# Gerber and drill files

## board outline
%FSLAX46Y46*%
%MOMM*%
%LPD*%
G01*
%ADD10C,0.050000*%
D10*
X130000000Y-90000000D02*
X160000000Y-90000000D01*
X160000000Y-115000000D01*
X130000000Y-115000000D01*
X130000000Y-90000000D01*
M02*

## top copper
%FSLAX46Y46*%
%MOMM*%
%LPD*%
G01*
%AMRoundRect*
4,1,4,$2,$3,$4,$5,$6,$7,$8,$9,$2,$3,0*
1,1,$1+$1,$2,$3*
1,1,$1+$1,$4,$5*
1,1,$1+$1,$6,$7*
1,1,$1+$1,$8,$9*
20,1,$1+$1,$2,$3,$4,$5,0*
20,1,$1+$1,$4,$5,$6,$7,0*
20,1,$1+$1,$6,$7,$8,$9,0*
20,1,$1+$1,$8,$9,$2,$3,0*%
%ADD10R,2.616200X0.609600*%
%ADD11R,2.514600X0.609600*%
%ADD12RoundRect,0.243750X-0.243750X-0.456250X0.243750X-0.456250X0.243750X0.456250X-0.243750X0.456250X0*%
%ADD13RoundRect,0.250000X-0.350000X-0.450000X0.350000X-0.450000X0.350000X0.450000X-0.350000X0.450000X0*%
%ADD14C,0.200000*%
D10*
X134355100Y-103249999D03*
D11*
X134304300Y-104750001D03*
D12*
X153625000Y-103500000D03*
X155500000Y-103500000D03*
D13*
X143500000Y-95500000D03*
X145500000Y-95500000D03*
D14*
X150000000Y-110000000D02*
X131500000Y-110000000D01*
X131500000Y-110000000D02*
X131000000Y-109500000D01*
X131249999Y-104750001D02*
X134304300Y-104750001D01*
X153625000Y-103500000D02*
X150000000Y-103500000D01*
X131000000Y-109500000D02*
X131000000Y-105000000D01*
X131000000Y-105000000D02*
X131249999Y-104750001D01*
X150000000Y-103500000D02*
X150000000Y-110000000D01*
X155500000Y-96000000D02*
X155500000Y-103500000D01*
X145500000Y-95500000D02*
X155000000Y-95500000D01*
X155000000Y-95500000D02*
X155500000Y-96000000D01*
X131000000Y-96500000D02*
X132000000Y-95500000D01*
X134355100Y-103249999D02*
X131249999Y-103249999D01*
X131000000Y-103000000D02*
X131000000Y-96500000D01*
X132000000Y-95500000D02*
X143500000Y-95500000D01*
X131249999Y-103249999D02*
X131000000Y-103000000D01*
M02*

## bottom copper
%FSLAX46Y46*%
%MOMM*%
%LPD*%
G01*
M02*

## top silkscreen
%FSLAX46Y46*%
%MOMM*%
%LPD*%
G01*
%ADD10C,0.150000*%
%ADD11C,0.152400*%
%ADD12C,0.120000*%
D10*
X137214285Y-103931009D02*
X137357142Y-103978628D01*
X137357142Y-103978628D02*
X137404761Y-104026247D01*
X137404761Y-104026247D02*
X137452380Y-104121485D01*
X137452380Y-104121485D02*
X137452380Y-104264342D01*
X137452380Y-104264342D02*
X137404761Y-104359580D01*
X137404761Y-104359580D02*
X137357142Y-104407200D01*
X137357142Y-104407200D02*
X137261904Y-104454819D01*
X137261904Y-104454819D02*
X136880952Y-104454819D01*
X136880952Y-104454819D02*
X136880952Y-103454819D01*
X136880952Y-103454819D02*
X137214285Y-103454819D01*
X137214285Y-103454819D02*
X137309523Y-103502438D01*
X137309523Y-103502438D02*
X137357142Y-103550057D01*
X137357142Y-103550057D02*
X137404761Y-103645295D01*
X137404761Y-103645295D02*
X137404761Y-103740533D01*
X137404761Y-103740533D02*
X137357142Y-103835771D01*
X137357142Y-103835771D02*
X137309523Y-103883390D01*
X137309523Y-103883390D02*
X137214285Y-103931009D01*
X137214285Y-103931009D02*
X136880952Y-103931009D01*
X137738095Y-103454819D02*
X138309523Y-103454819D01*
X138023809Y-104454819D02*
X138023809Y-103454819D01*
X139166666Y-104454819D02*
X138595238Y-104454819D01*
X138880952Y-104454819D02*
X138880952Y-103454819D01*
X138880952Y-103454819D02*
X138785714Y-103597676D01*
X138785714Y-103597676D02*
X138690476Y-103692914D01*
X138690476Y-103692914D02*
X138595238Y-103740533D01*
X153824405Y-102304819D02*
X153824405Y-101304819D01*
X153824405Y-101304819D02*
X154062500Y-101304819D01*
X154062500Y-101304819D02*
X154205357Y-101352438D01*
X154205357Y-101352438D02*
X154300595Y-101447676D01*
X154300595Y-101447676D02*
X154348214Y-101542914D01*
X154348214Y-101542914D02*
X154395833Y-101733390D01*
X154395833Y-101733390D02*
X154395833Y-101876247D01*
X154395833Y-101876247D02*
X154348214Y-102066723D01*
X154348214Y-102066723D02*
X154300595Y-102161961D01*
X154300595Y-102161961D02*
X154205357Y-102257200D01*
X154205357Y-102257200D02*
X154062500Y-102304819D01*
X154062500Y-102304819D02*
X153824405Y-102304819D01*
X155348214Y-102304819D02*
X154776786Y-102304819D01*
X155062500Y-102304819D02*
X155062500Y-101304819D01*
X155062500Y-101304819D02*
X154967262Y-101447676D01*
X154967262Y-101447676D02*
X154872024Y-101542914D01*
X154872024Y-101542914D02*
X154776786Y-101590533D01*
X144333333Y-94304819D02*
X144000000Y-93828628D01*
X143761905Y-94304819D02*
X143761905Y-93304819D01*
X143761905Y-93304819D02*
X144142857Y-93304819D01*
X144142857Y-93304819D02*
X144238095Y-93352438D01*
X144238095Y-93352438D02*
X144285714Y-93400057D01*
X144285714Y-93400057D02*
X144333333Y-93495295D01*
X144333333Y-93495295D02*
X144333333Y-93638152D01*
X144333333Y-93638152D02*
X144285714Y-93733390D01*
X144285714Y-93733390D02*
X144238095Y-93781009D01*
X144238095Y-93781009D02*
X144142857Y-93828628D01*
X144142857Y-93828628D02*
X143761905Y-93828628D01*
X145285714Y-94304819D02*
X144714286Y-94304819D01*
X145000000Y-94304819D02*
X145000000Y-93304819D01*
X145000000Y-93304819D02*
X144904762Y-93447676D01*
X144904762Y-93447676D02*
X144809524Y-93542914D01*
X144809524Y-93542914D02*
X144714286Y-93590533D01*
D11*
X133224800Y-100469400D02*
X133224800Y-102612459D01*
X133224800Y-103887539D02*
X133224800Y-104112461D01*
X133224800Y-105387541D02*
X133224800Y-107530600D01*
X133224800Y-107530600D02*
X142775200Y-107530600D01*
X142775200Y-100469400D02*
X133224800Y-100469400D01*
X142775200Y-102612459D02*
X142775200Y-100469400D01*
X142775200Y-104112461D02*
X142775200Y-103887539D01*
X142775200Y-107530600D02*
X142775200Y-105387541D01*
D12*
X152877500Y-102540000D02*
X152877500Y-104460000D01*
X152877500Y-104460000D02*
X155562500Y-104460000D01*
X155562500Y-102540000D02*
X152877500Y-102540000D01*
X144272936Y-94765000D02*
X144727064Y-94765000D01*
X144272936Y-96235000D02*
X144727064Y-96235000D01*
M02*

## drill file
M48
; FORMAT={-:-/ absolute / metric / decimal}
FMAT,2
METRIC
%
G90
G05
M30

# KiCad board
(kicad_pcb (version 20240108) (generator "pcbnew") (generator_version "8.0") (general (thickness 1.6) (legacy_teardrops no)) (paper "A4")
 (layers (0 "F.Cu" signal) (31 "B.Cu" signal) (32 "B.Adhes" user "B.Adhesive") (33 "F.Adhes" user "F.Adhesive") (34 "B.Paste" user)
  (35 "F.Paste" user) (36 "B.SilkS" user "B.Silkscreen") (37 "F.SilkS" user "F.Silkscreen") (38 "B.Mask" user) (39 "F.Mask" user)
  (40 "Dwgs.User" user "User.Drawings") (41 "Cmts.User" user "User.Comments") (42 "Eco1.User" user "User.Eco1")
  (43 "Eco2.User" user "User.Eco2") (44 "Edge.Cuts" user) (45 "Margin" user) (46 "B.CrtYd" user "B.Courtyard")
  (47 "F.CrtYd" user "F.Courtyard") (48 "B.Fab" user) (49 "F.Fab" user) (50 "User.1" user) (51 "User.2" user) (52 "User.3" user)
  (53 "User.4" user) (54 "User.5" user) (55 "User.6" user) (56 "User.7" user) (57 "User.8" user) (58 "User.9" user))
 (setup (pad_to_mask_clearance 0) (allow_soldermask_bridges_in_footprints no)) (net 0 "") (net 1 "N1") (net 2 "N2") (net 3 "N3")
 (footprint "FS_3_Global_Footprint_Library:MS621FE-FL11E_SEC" (layer "F.Cu") (at 138 104)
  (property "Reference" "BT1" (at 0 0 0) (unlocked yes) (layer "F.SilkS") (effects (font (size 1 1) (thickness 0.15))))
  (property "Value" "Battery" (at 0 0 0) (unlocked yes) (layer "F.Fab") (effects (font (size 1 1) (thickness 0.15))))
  (fp_line (start -4.7752 -3.5306) (end -4.7752 -1.387541) (stroke (width 0.1524) (type solid)) (layer "F.SilkS"))
  (fp_line (start -4.7752 -0.112461) (end -4.7752 0.112461) (stroke (width 0.1524) (type solid)) (layer "F.SilkS"))
  (fp_line (start -4.7752 1.387541) (end -4.7752 3.5306) (stroke (width 0.1524) (type solid)) (layer "F.SilkS"))
  (fp_line (start -4.7752 3.5306) (end 4.7752 3.5306) (stroke (width 0.1524) (type solid)) (layer "F.SilkS"))
  (fp_line (start 4.7752 -3.5306) (end -4.7752 -3.5306) (stroke (width 0.1524) (type solid)) (layer "F.SilkS"))
  (fp_line (start 4.7752 -1.387541) (end 4.7752 -3.5306) (stroke (width 0.1524) (type solid)) (layer "F.SilkS"))
  (fp_line (start 4.7752 0.112461) (end 4.7752 -0.112461) (stroke (width 0.1524) (type solid)) (layer "F.SilkS"))
  (fp_line (start 4.7752 3.5306) (end 4.7752 1.387541) (stroke (width 0.1524) (type solid)) (layer "F.SilkS"))
  (pad "1" smd rect (at -3.6449 -0.750001) (size 2.6162 0.6096) (layers "F.Cu" "F.Paste" "F.Mask") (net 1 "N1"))
  (pad "2" smd rect (at -3.6957 0.750001) (size 2.5146 0.6096) (layers "F.Cu" "F.Paste" "F.Mask") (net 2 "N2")))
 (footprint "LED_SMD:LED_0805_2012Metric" (layer "F.Cu") (at 154.5625 103.5)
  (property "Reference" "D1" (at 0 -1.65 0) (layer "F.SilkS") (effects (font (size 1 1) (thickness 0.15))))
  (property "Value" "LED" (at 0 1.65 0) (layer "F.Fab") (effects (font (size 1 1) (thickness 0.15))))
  (fp_line (start -1.685 -0.96) (end -1.685 0.96) (stroke (width 0.12) (type solid)) (layer "F.SilkS"))
  (fp_line (start -1.685 0.96) (end 1 0.96) (stroke (width 0.12) (type solid)) (layer "F.SilkS"))
  (fp_line (start 1 -0.96) (end -1.685 -0.96) (stroke (width 0.12) (type solid)) (layer "F.SilkS"))
  (pad "1" smd roundrect (at -0.9375 0) (size 0.975 1.4) (layers "F.Cu" "F.Paste" "F.Mask") (roundrect_rratio 0.25) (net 2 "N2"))
  (pad "2" smd roundrect (at 0.9375 0) (size 0.975 1.4) (layers "F.Cu" "F.Paste" "F.Mask") (roundrect_rratio 0.25) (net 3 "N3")))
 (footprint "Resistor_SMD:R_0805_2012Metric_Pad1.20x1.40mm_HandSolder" (layer "F.Cu") (at 144.5 95.5)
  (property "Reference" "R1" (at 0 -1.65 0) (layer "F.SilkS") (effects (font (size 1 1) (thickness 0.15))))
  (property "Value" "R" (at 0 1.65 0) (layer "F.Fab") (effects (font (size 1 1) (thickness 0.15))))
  (fp_line (start -0.227064 -0.735) (end 0.227064 -0.735) (stroke (width 0.12) (type solid)) (layer "F.SilkS"))
  (fp_line (start -0.227064 0.735) (end 0.227064 0.735) (stroke (width 0.12) (type solid)) (layer "F.SilkS"))
  (pad "1" smd roundrect (at -1 0) (size 1.2 1.4) (layers "F.Cu" "F.Paste" "F.Mask") (roundrect_rratio 0.208333) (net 1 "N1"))
  (pad "2" smd roundrect (at 1 0) (size 1.2 1.4) (layers "F.Cu" "F.Paste" "F.Mask") (roundrect_rratio 0.208333) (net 3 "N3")))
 (gr_rect (start 130 90) (end 160 115) (stroke (width 0.05) (type default)) (fill none) (layer "Edge.Cuts"))
 (segment (start 150 110) (end 131.5 110) (width 0.2) (layer "F.Cu") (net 2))
 (segment (start 131.5 110) (end 131 109.5) (width 0.2) (layer "F.Cu") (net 2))
 (segment (start 131.249999 104.750001) (end 134.3043 104.750001) (width 0.2) (layer "F.Cu") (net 2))
 (segment (start 153.625 103.5) (end 150 103.5) (width 0.2) (layer "F.Cu") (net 2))
 (segment (start 131 109.5) (end 131 105) (width 0.2) (layer "F.Cu") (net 2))
 (segment (start 131 105) (end 131.249999 104.750001) (width 0.2) (layer "F.Cu") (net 2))
 (segment (start 150 103.5) (end 150 110) (width 0.2) (layer "F.Cu") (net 2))
 (segment (start 155.5 96) (end 155.5 103.5) (width 0.2) (layer "F.Cu") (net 3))
 (segment (start 145.5 95.5) (end 155 95.5) (width 0.2) (layer "F.Cu") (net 3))
 (segment (start 155 95.5) (end 155.5 96) (width 0.2) (layer "F.Cu") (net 3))
 (segment (start 131 96.5) (end 132 95.5) (width 0.2) (layer "F.Cu") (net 1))
 (segment (start 134.3551 103.249999) (end 131.249999 103.249999) (width 0.2) (layer "F.Cu") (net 1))
 (segment (start 131 103) (end 131 96.5) (width 0.2) (layer "F.Cu") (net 1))
 (segment (start 132 95.5) (end 143.5 95.5) (width 0.2) (layer "F.Cu") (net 1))
 (segment (start 131.249999 103.249999) (end 131 103) (width 0.2) (layer "F.Cu") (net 1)))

